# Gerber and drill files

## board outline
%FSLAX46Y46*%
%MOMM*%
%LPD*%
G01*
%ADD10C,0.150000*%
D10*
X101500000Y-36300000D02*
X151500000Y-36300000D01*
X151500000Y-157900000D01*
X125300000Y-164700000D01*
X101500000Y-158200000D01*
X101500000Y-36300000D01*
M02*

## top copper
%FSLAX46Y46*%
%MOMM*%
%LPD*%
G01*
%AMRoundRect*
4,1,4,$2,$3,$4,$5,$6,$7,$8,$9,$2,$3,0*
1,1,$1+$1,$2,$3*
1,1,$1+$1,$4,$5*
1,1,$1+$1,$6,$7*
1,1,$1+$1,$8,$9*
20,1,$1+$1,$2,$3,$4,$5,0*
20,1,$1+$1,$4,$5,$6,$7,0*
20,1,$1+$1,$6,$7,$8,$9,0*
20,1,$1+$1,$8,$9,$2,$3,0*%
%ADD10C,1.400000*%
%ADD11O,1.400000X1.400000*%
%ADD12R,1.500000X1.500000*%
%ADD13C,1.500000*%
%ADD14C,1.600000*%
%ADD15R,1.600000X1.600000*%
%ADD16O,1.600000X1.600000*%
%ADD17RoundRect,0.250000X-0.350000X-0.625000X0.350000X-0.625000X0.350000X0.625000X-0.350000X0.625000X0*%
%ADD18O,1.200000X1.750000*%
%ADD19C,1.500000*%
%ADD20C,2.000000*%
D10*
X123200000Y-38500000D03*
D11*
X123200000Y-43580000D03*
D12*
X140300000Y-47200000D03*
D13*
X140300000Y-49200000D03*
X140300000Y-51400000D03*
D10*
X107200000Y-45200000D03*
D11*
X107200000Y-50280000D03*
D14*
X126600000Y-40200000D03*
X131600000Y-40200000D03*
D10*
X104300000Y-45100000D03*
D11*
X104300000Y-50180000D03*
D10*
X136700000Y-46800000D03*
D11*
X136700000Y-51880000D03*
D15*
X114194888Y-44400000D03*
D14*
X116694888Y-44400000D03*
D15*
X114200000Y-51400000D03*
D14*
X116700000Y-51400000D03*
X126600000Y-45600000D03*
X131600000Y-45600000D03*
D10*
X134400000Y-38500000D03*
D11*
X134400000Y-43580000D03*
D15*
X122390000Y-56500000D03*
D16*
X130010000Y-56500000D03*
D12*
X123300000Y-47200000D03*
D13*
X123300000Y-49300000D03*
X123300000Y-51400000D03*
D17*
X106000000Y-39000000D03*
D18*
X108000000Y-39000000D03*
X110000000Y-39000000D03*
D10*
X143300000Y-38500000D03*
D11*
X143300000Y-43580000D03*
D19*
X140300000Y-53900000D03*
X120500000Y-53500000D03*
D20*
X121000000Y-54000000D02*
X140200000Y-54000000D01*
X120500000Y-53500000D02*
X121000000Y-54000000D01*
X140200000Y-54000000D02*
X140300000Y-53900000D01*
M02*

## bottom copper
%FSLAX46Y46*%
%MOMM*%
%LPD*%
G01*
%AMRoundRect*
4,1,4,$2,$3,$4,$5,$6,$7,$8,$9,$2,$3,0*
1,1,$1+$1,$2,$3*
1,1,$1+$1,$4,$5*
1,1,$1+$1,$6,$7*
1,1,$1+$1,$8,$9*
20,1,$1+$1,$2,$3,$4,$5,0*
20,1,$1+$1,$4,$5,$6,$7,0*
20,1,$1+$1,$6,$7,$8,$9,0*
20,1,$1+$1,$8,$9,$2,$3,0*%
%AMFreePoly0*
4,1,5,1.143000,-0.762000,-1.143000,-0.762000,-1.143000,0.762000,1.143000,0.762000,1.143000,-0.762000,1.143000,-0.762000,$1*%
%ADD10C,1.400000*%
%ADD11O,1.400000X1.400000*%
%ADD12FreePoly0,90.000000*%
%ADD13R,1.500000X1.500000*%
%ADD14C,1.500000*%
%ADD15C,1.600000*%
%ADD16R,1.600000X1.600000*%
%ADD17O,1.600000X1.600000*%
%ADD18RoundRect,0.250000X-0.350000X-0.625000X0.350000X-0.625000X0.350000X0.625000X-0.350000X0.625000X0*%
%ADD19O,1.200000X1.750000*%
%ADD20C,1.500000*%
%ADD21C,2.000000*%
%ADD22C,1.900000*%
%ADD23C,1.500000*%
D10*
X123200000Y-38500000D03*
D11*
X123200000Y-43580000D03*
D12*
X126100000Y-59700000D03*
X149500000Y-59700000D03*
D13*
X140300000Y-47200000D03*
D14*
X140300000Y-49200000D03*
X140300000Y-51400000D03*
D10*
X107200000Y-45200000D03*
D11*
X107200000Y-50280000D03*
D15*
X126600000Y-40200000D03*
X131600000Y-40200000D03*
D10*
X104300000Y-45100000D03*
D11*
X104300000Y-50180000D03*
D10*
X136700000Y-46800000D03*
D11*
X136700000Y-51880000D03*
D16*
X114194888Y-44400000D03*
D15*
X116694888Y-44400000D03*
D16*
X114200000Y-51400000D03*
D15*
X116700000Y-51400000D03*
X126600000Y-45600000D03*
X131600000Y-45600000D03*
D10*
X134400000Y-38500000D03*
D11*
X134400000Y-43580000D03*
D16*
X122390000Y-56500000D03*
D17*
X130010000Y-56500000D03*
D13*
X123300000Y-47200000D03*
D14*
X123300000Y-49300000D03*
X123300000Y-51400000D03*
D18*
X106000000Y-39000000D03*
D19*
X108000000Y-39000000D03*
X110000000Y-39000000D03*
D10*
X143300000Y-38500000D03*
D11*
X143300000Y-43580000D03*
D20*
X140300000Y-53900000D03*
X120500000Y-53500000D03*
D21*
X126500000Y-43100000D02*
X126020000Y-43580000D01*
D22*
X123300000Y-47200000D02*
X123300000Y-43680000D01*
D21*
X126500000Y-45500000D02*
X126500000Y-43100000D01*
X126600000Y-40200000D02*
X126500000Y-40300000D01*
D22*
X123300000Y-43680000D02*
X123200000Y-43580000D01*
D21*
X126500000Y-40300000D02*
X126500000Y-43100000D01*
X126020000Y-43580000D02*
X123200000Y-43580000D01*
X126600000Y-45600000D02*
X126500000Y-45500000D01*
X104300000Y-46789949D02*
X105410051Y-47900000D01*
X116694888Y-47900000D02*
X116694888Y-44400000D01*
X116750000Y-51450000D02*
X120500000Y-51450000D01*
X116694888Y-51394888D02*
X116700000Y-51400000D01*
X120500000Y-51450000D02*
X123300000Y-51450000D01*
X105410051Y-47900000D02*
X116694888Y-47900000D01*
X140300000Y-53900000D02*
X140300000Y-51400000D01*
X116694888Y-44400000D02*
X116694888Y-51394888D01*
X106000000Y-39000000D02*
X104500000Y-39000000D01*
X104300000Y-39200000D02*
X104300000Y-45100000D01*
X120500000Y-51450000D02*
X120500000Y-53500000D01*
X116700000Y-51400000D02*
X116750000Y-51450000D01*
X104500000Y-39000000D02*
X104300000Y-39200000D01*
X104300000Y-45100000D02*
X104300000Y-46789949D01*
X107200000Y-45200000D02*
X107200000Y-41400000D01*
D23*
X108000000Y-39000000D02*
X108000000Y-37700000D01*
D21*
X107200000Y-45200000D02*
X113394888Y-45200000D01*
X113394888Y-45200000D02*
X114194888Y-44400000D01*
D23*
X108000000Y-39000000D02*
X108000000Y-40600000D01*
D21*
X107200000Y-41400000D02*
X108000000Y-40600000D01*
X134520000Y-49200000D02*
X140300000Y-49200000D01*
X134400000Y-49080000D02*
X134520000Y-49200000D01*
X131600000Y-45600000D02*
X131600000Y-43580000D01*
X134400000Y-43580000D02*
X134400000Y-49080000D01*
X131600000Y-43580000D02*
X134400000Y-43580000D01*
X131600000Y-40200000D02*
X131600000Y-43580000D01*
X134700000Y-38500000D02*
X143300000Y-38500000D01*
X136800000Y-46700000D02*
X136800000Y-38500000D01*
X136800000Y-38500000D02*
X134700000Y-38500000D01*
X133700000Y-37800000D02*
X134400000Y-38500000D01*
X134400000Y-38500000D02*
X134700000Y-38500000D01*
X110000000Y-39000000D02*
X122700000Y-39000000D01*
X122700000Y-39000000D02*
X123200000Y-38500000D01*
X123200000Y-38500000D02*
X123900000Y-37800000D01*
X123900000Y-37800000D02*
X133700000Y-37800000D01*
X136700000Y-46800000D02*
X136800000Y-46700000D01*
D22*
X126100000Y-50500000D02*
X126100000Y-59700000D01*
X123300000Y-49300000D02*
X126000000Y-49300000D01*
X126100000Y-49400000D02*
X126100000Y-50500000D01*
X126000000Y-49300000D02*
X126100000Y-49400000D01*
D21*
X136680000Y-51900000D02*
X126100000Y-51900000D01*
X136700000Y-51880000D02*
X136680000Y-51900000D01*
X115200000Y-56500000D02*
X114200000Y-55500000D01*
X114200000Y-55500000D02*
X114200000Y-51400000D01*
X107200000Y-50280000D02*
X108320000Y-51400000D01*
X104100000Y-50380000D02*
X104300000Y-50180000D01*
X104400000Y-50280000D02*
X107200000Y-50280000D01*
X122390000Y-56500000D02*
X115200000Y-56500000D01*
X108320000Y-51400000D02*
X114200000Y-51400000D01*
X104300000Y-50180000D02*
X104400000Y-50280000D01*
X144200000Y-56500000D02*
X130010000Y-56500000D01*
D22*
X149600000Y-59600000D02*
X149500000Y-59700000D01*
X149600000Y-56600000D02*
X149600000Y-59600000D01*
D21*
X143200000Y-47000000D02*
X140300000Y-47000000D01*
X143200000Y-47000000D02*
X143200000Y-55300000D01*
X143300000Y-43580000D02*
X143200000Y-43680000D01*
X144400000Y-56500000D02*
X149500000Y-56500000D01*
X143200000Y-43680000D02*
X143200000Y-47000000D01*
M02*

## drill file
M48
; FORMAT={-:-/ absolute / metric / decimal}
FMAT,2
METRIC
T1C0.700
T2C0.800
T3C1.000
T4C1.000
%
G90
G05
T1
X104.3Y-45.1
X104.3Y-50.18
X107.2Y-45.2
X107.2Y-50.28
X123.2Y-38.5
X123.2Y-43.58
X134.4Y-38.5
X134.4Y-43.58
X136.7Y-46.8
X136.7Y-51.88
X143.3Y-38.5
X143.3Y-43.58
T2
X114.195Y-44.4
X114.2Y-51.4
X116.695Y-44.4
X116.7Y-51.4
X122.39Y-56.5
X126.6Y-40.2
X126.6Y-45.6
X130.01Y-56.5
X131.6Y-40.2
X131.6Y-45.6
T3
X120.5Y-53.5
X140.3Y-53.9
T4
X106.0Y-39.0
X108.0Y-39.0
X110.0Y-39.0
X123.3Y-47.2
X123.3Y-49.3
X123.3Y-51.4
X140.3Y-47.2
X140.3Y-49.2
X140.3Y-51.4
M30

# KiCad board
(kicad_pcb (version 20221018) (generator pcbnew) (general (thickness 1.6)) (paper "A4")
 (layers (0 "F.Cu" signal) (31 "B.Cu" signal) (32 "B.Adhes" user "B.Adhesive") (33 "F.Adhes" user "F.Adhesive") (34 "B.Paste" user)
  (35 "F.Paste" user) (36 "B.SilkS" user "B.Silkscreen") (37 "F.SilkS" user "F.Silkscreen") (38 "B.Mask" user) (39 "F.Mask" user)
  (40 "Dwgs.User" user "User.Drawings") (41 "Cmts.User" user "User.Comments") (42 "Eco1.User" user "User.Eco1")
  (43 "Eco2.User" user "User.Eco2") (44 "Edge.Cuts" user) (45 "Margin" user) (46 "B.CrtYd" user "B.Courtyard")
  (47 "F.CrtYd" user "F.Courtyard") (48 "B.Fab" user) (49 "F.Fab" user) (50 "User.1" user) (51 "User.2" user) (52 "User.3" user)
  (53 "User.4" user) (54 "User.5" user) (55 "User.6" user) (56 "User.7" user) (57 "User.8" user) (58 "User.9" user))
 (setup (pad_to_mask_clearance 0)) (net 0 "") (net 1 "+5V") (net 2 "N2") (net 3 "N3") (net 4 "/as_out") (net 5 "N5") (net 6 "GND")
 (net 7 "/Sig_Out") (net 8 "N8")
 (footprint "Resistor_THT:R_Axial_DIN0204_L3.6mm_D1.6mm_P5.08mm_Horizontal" (layer "F.Cu") (at 123.2 38.5 -90)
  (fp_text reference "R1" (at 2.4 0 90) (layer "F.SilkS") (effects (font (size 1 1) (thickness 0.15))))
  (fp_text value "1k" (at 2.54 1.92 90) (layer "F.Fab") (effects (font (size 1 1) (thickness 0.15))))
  (pad "1" thru_hole circle (at 0 0 270) (size 1.4 1.4) (drill 0.7) (layers "*.Cu" "*.Mask") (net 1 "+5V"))
  (pad "2" thru_hole oval (at 5.08 0 270) (size 1.4 1.4) (drill 0.7) (layers "*.Cu" "*.Mask") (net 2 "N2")))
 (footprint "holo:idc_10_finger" (layer "F.Cu") (at 114.3 68.5)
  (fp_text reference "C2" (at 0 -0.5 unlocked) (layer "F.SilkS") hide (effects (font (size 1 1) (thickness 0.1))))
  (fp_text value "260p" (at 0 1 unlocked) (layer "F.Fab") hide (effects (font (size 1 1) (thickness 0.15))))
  (pad "1" smd custom (at 11.8 -8.8 90) (size 2.286 1.524) (layers "B.Cu" "F.Paste" "F.Mask") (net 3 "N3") (thermal_bridge_angle 45)
   (options (clearance outline) (anchor rect)) (primitives))
  (pad "2" smd custom (at 35.2 -8.8 90) (size 2.286 1.524) (layers "B.Cu" "F.Paste" "F.Mask") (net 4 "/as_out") (thermal_bridge_angle 45)
   (options (clearance outline) (anchor rect)) (primitives)))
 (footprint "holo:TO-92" (layer "F.Cu") (at 140.3 48 -90)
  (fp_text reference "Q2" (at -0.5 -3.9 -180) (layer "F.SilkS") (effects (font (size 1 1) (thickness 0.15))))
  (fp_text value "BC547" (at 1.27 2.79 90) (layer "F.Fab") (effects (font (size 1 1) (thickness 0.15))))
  (pad "1" thru_hole rect (at -0.8 0 270) (size 1.5 1.5) (drill 1) (layers "*.Cu" "*.Mask") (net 4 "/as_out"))
  (pad "2" thru_hole circle (at 1.2 0 270) (size 1.5 1.5) (drill 1) (layers "*.Cu" "*.Mask") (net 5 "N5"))
  (pad "3" thru_hole circle (at 3.4 0 270) (size 1.5 1.5) (drill 1) (layers "*.Cu" "*.Mask") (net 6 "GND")))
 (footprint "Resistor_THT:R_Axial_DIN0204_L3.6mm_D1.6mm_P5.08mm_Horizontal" (layer "F.Cu") (at 107.2 45.2 -90)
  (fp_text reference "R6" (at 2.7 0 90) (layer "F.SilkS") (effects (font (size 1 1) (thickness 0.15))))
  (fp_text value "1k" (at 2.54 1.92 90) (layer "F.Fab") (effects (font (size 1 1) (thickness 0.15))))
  (pad "1" thru_hole circle (at 0 0 270) (size 1.4 1.4) (drill 0.7) (layers "*.Cu" "*.Mask") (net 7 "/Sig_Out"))
  (pad "2" thru_hole oval (at 5.08 0 270) (size 1.4 1.4) (drill 0.7) (layers "*.Cu" "*.Mask") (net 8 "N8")))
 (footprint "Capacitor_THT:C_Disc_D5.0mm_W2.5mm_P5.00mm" (layer "F.Cu") (at 126.6 40.2)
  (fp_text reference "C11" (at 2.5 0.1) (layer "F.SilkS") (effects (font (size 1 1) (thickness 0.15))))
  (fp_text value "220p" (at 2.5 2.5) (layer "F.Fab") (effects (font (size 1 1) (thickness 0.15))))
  (pad "1" thru_hole circle (at 0 0) (size 1.6 1.6) (drill 0.8) (layers "*.Cu" "*.Mask") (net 2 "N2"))
  (pad "2" thru_hole circle (at 5 0) (size 1.6 1.6) (drill 0.8) (layers "*.Cu" "*.Mask") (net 5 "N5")))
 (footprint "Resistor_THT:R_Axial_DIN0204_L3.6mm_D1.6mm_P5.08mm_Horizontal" (layer "F.Cu") (at 104.3 45.1 -90)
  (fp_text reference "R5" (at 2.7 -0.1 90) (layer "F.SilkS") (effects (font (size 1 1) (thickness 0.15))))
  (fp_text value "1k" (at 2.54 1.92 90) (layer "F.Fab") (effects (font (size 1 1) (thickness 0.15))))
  (pad "1" thru_hole circle (at 0 0 270) (size 1.4 1.4) (drill 0.7) (layers "*.Cu" "*.Mask") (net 6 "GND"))
  (pad "2" thru_hole oval (at 5.08 0 270) (size 1.4 1.4) (drill 0.7) (layers "*.Cu" "*.Mask") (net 8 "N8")))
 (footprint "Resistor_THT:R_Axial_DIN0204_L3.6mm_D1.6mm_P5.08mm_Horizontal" (layer "F.Cu") (at 136.7 46.8 -90)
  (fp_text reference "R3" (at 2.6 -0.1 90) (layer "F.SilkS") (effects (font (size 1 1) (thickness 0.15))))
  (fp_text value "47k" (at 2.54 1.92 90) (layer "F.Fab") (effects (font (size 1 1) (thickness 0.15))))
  (pad "1" thru_hole circle (at 0 0 270) (size 1.4 1.4) (drill 0.7) (layers "*.Cu" "*.Mask") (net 1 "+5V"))
  (pad "2" thru_hole oval (at 5.08 0 270) (size 1.4 1.4) (drill 0.7) (layers "*.Cu" "*.Mask") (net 3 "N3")))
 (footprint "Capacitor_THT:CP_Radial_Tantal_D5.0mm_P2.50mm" (layer "F.Cu") (at 114.194888 44.4)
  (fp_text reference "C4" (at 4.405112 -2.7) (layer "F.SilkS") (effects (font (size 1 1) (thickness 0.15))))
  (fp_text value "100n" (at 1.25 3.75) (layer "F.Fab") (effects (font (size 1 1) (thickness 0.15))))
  (pad "1" thru_hole rect (at 0 0) (size 1.6 1.6) (drill 0.8) (layers "*.Cu" "*.Mask") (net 7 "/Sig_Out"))
  (pad "2" thru_hole circle (at 2.5 0) (size 1.6 1.6) (drill 0.8) (layers "*.Cu" "*.Mask") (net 6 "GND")))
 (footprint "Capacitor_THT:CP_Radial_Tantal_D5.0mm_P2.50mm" (layer "F.Cu") (at 114.2 51.4)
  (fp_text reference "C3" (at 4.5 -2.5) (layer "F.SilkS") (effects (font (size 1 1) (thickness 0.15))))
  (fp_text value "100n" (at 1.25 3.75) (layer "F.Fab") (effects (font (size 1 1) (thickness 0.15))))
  (pad "1" thru_hole rect (at 0 0) (size 1.6 1.6) (drill 0.8) (layers "*.Cu" "*.Mask") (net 8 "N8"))
  (pad "2" thru_hole circle (at 2.5 0) (size 1.6 1.6) (drill 0.8) (layers "*.Cu" "*.Mask") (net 6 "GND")))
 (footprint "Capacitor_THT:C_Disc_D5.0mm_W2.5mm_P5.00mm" (layer "F.Cu") (at 126.6 45.6)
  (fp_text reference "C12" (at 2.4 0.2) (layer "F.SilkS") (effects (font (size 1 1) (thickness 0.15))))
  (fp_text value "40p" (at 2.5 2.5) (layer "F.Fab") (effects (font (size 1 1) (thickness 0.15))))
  (pad "1" thru_hole circle (at 0 0) (size 1.6 1.6) (drill 0.8) (layers "*.Cu" "*.Mask") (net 2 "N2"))
  (pad "2" thru_hole circle (at 5 0) (size 1.6 1.6) (drill 0.8) (layers "*.Cu" "*.Mask") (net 5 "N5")))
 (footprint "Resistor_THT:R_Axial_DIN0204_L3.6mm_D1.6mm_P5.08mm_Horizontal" (layer "F.Cu") (at 134.4 38.5 -90)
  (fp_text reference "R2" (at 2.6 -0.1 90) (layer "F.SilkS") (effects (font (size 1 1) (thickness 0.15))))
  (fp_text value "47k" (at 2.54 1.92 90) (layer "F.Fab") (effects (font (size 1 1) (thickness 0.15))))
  (pad "1" thru_hole circle (at 0 0 270) (size 1.4 1.4) (drill 0.7) (layers "*.Cu" "*.Mask") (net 1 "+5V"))
  (pad "2" thru_hole oval (at 5.08 0 270) (size 1.4 1.4) (drill 0.7) (layers "*.Cu" "*.Mask") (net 5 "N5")))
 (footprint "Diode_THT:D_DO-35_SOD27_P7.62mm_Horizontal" (layer "F.Cu") (at 122.39 56.5)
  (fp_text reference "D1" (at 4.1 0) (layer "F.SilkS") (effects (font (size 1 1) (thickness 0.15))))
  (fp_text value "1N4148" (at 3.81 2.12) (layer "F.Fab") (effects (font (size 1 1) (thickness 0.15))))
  (pad "1" thru_hole rect (at 0 0) (size 1.6 1.6) (drill 0.8) (layers "*.Cu" "*.Mask") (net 8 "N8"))
  (pad "2" thru_hole oval (at 7.62 0) (size 1.6 1.6) (drill 0.8) (layers "*.Cu" "*.Mask") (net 4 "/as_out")))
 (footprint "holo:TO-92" (layer "F.Cu") (at 123.3 48 -90)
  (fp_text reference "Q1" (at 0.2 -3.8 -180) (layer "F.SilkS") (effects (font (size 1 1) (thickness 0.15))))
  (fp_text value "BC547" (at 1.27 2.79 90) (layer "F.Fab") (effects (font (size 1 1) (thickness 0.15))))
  (pad "1" thru_hole rect (at -0.8 0 270) (size 1.5 1.5) (drill 1) (layers "*.Cu" "*.Mask") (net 2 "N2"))
  (pad "2" thru_hole circle (at 1.3 0 270) (size 1.5 1.5) (drill 1) (layers "*.Cu" "*.Mask") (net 3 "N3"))
  (pad "3" thru_hole circle (at 3.4 0 270) (size 1.5 1.5) (drill 1) (layers "*.Cu" "*.Mask") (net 6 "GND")))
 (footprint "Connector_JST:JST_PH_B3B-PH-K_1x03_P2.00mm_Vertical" (layer "F.Cu") (at 106 39)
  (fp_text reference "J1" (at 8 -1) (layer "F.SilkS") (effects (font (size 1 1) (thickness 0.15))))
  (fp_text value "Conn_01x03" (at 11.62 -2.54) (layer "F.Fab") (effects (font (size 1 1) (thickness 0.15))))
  (pad "1" thru_hole roundrect (at 0 0) (size 1.2 1.75) (drill 1) (layers "*.Cu" "*.Mask") (roundrect_rratio 0.208333) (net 6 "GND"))
  (pad "2" thru_hole oval (at 2 0) (size 1.2 1.75) (drill 1) (layers "*.Cu" "*.Mask") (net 7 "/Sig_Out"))
  (pad "3" thru_hole oval (at 4 0) (size 1.2 1.75) (drill 1) (layers "*.Cu" "*.Mask") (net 1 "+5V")))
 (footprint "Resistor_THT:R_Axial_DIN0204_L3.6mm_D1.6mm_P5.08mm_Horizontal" (layer "F.Cu") (at 143.3 38.5 -90)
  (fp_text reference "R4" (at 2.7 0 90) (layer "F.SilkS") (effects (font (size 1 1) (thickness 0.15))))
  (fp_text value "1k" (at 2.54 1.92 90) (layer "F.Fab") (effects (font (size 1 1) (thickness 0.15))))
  (pad "1" thru_hole circle (at 0 0 270) (size 1.4 1.4) (drill 0.7) (layers "*.Cu" "*.Mask") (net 1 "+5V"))
  (pad "2" thru_hole oval (at 5.08 0 270) (size 1.4 1.4) (drill 0.7) (layers "*.Cu" "*.Mask") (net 4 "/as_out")))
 (gr_poly
  (pts (xy 101.5 36.3) (xy 151.5 36.3) (xy 151.5 157.9) (xy 125.3 164.7) (xy 101.5 158.2)) (stroke (width 0.15) (type solid)) (fill none)
  (layer "Edge.Cuts"))
 (segment (start 126.5 43.1) (end 126.02 43.58) (width 2) (layer "B.Cu") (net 2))
 (segment (start 123.3 47.2) (end 123.3 43.68) (width 1.9) (layer "B.Cu") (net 2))
 (segment (start 126.5 45.5) (end 126.5 43.1) (width 2) (layer "B.Cu") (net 2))
 (segment (start 126.6 40.2) (end 126.5 40.3) (width 2) (layer "B.Cu") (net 2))
 (segment (start 123.3 43.68) (end 123.2 43.58) (width 1.9) (layer "B.Cu") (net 2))
 (segment (start 126.5 40.3) (end 126.5 43.1) (width 2) (layer "B.Cu") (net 2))
 (segment (start 126.02 43.58) (end 123.2 43.58) (width 2) (layer "B.Cu") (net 2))
 (segment (start 126.6 45.6) (end 126.5 45.5) (width 2) (layer "B.Cu") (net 2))
 (segment (start 121 54) (end 140.2 54) (width 2) (layer "F.Cu") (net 6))
 (segment (start 120.5 53.5) (end 121 54) (width 2) (layer "F.Cu") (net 6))
 (segment (start 140.2 54) (end 140.3 53.9) (width 2) (layer "F.Cu") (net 6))
 (via (at 140.3 53.9) (size 1.5) (drill 1) (layers "F.Cu" "B.Cu") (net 6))
 (via (at 120.5 53.5) (size 1.5) (drill 1) (layers "F.Cu" "B.Cu") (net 6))
 (segment (start 104.3 46.789949) (end 105.410051 47.9) (width 2) (layer "B.Cu") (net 6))
 (segment (start 116.694888 47.9) (end 116.694888 44.4) (width 2) (layer "B.Cu") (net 6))
 (segment (start 116.75 51.45) (end 120.5 51.45) (width 2) (layer "B.Cu") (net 6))
 (segment (start 116.694888 51.394888) (end 116.7 51.4) (width 2) (layer "B.Cu") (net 6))
 (segment (start 120.5 51.45) (end 123.3 51.45) (width 2) (layer "B.Cu") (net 6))
 (segment (start 105.410051 47.9) (end 116.694888 47.9) (width 2) (layer "B.Cu") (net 6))
 (segment (start 140.3 53.9) (end 140.3 51.4) (width 2) (layer "B.Cu") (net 6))
 (segment (start 116.694888 44.4) (end 116.694888 51.394888) (width 2) (layer "B.Cu") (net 6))
 (segment (start 106 39) (end 104.5 39) (width 2) (layer "B.Cu") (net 6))
 (segment (start 104.3 39.2) (end 104.3 45.1) (width 2) (layer "B.Cu") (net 6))
 (segment (start 120.5 51.45) (end 120.5 53.5) (width 2) (layer "B.Cu") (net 6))
 (segment (start 116.7 51.4) (end 116.75 51.45) (width 2) (layer "B.Cu") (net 6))
 (segment (start 104.5 39) (end 104.3 39.2) (width 2) (layer "B.Cu") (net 6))
 (segment (start 104.3 45.1) (end 104.3 46.789949) (width 2) (layer "B.Cu") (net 6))
 (segment (start 107.2 45.2) (end 107.2 41.4) (width 2) (layer "B.Cu") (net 7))
 (segment (start 108 39) (end 108 37.7) (width 1.5) (layer "B.Cu") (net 7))
 (segment (start 107.2 45.2) (end 113.394888 45.2) (width 2) (layer "B.Cu") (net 7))
 (segment (start 113.394888 45.2) (end 114.194888 44.4) (width 2) (layer "B.Cu") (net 7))
 (segment (start 108 39) (end 108 40.6) (width 1.5) (layer "B.Cu") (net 7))
 (segment (start 107.2 41.4) (end 108 40.6) (width 2) (layer "B.Cu") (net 7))
 (segment (start 134.52 49.2) (end 140.3 49.2) (width 2) (layer "B.Cu") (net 5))
 (segment (start 134.4 49.08) (end 134.52 49.2) (width 2) (layer "B.Cu") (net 5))
 (segment (start 131.6 45.6) (end 131.6 43.58) (width 2) (layer "B.Cu") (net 5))
 (segment (start 134.4 43.58) (end 134.4 49.08) (width 2) (layer "B.Cu") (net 5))
 (segment (start 131.6 43.58) (end 134.4 43.58) (width 2) (layer "B.Cu") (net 5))
 (segment (start 131.6 40.2) (end 131.6 43.58) (width 2) (layer "B.Cu") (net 5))
 (segment (start 134.7 38.5) (end 143.3 38.5) (width 2) (layer "B.Cu") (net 1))
 (segment (start 136.8 46.7) (end 136.8 38.5) (width 2) (layer "B.Cu") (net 1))
 (segment (start 136.8 38.5) (end 134.7 38.5) (width 2) (layer "B.Cu") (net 1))
 (segment (start 133.7 37.8) (end 134.4 38.5) (width 2) (layer "B.Cu") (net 1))
 (segment (start 134.4 38.5) (end 134.7 38.5) (width 2) (layer "B.Cu") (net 1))
 (segment (start 110 39) (end 122.7 39) (width 2) (layer "B.Cu") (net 1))
 (segment (start 122.7 39) (end 123.2 38.5) (width 2) (layer "B.Cu") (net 1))
 (segment (start 123.2 38.5) (end 123.9 37.8) (width 2) (layer "B.Cu") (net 1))
 (segment (start 123.9 37.8) (end 133.7 37.8) (width 2) (layer "B.Cu") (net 1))
 (segment (start 136.7 46.8) (end 136.8 46.7) (width 2) (layer "B.Cu") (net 1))
 (segment (start 126.1 50.5) (end 126.1 59.7) (width 1.9) (layer "B.Cu") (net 3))
 (segment (start 123.3 49.3) (end 126 49.3) (width 1.9) (layer "B.Cu") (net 3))
 (segment (start 126.1 49.4) (end 126.1 50.5) (width 1.9) (layer "B.Cu") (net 3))
 (segment (start 126 49.3) (end 126.1 49.4) (width 1.9) (layer "B.Cu") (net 3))
 (segment (start 136.68 51.9) (end 126.1 51.9) (width 2) (layer "B.Cu") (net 3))
 (segment (start 136.7 51.88) (end 136.68 51.9) (width 2) (layer "B.Cu") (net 3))
 (segment (start 115.2 56.5) (end 114.2 55.5) (width 2) (layer "B.Cu") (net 8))
 (segment (start 114.2 55.5) (end 114.2 51.4) (width 2) (layer "B.Cu") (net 8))
 (segment (start 107.2 50.28) (end 108.32 51.4) (width 2) (layer "B.Cu") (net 8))
 (segment (start 104.1 50.38) (end 104.3 50.18) (width 2) (layer "B.Cu") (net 8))
 (segment (start 104.4 50.28) (end 107.2 50.28) (width 2) (layer "B.Cu") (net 8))
 (segment (start 122.39 56.5) (end 115.2 56.5) (width 2) (layer "B.Cu") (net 8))
 (segment (start 108.32 51.4) (end 114.2 51.4) (width 2) (layer "B.Cu") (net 8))
 (segment (start 104.3 50.18) (end 104.4 50.28) (width 2) (layer "B.Cu") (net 8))
 (segment (start 144.2 56.5) (end 130.01 56.5) (width 2) (layer "B.Cu") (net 4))
 (segment (start 149.6 59.6) (end 149.5 59.7) (width 1.9) (layer "B.Cu") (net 4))
 (segment (start 149.6 56.6) (end 149.6 59.6) (width 1.9) (layer "B.Cu") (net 4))
 (segment (start 143.2 47) (end 140.3 47) (width 2) (layer "B.Cu") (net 4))
 (segment (start 143.2 47) (end 143.2 55.3) (width 2) (layer "B.Cu") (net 4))
 (segment (start 143.3 43.58) (end 143.2 43.68) (width 2) (layer "B.Cu") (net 4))
 (segment (start 144.4 56.5) (end 149.5 56.5) (width 2) (layer "B.Cu") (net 4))
 (segment (start 143.2 43.68) (end 143.2 47) (width 2) (layer "B.Cu") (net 4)))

